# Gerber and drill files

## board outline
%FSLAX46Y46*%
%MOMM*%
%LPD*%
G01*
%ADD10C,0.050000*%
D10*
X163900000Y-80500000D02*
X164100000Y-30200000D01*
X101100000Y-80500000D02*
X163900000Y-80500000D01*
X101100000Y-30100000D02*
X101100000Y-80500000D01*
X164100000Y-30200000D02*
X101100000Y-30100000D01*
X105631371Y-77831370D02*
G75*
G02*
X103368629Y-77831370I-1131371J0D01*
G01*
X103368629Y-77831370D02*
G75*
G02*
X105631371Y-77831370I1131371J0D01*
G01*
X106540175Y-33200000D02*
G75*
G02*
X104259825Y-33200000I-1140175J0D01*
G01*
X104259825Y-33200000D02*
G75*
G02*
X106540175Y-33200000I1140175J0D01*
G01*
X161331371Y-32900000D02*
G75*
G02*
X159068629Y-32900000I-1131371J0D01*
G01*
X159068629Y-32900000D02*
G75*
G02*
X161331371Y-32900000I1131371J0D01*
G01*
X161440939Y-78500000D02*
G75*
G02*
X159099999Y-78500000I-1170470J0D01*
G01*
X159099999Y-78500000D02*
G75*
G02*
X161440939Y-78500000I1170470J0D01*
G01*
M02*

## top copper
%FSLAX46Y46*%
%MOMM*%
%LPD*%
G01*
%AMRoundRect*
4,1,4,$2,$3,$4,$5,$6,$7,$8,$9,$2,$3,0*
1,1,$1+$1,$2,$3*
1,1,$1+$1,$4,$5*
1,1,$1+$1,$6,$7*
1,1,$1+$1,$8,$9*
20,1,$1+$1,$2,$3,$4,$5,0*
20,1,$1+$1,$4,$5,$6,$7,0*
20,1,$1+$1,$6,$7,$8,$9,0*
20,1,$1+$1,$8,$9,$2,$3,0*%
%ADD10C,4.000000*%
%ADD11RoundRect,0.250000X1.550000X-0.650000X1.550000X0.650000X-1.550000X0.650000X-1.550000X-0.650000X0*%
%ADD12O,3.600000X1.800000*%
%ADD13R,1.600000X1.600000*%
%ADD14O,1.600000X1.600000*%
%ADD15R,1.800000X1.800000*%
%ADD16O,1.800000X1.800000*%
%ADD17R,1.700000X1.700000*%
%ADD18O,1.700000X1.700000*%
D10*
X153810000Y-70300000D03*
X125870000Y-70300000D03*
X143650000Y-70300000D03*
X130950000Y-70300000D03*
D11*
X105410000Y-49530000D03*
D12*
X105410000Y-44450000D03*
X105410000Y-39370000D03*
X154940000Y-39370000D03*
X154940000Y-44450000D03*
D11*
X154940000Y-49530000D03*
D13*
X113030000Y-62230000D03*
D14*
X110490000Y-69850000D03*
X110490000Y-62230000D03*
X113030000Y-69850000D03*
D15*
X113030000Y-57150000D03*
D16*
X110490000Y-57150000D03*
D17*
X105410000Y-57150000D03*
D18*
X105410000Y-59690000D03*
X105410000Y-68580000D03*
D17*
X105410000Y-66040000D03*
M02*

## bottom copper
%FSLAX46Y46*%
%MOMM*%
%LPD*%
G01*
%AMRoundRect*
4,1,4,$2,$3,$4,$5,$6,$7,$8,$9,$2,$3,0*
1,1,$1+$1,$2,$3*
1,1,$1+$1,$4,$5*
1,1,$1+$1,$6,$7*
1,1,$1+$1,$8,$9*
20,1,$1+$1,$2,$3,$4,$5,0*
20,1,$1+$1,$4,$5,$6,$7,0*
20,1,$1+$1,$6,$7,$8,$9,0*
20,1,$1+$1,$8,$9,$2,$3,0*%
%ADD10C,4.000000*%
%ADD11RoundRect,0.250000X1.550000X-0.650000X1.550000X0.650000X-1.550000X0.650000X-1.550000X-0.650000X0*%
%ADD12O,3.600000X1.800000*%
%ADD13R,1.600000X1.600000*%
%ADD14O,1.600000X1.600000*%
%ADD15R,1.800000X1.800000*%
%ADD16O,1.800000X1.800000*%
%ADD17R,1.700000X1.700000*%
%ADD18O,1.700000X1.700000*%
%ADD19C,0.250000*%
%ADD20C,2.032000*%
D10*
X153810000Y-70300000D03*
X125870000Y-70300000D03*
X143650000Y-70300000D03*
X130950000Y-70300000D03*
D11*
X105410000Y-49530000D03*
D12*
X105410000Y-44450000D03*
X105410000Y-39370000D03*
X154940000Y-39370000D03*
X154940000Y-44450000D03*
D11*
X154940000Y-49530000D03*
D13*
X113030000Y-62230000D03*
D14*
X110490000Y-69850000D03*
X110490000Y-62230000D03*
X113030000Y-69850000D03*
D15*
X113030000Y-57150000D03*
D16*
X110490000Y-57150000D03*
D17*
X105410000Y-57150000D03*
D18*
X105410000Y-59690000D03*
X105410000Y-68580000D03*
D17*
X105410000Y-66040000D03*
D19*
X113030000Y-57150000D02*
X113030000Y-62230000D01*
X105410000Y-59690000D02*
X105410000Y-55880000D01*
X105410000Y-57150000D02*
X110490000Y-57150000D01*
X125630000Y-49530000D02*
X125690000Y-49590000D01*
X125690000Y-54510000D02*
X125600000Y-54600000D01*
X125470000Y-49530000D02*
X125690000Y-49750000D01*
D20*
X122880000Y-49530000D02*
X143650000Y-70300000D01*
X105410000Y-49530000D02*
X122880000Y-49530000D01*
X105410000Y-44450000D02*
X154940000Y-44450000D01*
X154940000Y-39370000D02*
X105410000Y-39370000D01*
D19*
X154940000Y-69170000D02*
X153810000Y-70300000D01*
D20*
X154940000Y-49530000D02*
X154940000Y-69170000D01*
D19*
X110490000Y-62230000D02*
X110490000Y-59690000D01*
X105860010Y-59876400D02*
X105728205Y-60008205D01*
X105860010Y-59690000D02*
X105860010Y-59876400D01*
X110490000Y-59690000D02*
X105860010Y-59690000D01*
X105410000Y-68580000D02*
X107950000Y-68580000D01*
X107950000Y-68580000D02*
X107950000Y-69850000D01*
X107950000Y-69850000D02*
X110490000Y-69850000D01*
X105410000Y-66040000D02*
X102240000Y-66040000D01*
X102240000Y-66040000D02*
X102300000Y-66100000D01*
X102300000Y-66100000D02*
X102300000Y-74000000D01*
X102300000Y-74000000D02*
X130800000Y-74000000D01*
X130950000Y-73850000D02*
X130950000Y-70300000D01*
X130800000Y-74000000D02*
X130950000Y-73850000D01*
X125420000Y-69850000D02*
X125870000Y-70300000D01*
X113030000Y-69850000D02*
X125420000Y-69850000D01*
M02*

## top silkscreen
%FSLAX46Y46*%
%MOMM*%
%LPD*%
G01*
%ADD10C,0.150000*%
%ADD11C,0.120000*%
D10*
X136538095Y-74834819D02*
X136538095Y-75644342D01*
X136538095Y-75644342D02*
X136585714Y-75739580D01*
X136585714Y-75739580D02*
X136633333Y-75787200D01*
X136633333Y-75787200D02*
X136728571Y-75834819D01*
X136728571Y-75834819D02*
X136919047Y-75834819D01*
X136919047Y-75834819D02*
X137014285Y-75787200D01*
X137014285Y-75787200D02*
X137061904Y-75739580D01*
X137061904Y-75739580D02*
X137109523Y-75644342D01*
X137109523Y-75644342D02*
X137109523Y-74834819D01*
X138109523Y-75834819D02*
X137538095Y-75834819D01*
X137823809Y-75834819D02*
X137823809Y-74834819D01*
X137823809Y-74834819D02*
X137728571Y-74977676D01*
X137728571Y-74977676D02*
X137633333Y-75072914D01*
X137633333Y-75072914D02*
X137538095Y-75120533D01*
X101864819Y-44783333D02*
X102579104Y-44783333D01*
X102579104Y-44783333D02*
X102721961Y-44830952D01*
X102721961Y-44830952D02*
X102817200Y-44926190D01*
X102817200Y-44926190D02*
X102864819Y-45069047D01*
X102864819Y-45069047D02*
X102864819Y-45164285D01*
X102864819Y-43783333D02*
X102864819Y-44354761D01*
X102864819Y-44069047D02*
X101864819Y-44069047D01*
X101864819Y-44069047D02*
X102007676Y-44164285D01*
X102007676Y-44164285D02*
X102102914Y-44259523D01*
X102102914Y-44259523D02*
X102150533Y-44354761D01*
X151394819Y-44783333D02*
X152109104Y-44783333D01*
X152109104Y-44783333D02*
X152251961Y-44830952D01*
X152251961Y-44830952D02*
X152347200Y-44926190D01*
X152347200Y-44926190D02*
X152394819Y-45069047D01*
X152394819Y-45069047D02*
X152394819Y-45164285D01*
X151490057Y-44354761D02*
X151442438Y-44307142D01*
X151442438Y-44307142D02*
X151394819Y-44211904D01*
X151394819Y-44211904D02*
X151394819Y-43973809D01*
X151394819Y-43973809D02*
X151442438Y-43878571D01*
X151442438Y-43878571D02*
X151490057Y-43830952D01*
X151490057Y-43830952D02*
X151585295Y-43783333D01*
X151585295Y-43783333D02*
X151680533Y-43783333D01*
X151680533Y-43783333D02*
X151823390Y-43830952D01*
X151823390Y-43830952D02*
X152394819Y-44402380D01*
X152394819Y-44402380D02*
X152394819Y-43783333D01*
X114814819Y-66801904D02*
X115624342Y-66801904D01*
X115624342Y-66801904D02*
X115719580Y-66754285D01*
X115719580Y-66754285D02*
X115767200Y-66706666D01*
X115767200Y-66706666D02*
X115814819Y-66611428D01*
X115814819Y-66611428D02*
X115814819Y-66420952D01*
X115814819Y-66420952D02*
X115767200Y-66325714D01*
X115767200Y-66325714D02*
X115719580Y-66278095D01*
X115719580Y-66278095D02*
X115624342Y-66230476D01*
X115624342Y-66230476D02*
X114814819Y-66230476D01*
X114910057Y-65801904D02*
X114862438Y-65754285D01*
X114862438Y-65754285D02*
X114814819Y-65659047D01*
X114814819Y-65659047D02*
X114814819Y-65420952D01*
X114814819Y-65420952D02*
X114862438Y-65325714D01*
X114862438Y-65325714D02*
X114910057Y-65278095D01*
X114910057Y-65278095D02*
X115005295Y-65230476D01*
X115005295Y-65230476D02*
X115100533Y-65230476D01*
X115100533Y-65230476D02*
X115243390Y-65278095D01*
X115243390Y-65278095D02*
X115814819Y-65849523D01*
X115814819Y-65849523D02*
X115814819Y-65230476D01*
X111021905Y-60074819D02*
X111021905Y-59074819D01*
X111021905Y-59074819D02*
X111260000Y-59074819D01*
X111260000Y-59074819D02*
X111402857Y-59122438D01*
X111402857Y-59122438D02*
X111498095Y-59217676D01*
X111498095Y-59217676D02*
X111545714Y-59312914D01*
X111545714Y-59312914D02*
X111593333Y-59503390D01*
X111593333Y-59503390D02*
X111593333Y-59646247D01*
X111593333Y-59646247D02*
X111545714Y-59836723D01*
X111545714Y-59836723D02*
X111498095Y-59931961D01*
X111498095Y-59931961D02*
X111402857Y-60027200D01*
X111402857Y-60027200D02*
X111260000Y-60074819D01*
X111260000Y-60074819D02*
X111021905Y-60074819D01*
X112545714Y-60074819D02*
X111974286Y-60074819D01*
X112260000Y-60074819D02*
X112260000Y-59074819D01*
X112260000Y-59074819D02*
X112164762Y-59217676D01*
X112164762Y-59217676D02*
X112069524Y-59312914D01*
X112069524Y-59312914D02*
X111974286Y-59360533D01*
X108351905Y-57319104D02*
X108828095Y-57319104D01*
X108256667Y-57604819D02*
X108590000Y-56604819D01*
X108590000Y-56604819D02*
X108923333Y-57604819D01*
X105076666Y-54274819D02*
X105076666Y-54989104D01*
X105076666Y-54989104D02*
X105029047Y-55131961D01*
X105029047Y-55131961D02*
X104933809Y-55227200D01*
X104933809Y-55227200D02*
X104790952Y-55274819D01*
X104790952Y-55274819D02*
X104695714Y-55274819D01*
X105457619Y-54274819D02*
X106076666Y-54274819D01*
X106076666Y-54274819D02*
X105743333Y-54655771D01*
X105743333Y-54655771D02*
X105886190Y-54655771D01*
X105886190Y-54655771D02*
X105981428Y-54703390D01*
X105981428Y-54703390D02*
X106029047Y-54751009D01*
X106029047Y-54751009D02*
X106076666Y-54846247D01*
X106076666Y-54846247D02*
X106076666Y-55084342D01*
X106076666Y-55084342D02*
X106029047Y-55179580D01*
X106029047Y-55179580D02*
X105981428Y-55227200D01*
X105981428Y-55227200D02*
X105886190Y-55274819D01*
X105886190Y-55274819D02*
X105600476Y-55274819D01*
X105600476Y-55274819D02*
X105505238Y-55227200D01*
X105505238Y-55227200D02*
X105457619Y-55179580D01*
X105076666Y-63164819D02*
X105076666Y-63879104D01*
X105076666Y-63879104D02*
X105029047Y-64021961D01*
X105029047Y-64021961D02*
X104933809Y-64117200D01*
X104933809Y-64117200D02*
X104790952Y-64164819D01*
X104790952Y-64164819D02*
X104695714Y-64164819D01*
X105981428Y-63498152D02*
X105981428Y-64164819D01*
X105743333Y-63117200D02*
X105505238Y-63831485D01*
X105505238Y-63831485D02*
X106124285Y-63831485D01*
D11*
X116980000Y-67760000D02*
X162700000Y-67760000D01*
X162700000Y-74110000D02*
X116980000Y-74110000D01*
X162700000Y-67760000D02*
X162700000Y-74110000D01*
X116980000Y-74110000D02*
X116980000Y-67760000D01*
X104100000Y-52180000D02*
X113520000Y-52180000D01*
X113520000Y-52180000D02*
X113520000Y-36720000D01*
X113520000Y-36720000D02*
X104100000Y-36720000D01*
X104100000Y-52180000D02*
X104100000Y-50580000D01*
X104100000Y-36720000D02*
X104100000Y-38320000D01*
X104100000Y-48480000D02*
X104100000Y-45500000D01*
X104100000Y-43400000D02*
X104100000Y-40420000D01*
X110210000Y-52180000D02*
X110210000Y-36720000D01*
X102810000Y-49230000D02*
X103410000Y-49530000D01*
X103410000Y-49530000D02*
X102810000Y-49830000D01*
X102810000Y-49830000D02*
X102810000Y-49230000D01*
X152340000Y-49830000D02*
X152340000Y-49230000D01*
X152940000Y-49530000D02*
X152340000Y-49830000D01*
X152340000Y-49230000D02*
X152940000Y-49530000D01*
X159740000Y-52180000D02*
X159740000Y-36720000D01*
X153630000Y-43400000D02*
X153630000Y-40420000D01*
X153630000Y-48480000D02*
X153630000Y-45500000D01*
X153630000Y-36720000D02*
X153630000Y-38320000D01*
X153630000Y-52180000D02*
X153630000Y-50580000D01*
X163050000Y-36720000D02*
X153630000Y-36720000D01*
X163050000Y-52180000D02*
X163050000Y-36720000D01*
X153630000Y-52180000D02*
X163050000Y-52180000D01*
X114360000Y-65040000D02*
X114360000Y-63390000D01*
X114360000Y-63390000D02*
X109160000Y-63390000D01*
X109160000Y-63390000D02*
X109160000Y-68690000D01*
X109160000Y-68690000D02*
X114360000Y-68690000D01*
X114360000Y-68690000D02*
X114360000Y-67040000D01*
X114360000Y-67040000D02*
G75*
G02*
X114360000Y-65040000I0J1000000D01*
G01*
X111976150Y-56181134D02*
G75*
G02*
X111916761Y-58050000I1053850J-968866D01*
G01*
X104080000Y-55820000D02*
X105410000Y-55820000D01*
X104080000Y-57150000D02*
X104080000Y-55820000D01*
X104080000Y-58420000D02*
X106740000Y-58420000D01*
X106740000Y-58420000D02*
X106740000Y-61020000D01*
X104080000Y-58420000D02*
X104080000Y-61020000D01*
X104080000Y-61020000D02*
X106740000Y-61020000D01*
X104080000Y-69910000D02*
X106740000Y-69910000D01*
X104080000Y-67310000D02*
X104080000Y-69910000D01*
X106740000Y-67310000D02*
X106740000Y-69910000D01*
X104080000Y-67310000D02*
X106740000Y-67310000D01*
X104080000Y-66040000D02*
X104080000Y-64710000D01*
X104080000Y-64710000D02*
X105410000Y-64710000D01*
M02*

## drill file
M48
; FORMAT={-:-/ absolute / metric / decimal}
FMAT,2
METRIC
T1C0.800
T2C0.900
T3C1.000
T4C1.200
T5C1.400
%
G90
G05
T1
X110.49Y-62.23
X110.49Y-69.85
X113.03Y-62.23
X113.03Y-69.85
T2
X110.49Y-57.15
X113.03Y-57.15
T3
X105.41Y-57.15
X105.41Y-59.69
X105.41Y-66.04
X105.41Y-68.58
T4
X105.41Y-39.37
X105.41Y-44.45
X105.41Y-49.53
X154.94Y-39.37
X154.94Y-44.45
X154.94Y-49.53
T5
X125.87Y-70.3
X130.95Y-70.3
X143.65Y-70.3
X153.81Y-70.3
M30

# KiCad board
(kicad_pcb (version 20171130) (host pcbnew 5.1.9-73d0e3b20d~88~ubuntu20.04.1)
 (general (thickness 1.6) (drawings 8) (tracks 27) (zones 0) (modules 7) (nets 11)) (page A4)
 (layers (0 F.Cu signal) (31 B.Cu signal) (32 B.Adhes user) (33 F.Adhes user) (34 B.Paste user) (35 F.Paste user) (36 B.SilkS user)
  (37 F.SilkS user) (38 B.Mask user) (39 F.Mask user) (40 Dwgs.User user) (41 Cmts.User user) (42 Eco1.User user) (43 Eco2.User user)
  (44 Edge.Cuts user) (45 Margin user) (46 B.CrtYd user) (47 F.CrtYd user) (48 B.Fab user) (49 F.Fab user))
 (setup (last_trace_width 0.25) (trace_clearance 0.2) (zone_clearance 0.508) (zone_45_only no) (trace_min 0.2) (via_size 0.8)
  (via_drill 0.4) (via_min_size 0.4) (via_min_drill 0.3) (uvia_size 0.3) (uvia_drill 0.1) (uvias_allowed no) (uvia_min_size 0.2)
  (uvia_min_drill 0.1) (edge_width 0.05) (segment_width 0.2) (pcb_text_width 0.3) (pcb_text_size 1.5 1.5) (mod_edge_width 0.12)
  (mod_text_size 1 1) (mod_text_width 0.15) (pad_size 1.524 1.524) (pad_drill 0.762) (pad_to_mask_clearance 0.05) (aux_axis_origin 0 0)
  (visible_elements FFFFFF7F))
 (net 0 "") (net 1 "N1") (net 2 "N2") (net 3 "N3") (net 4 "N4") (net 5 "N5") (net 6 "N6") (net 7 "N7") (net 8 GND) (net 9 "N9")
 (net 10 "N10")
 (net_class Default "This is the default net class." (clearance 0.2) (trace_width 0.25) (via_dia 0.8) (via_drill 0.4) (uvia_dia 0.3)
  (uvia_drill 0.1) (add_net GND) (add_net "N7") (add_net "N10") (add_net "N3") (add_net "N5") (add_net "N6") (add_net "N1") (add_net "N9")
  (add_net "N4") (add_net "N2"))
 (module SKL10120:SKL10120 (layer F.Cu) (at 137.3 70.3)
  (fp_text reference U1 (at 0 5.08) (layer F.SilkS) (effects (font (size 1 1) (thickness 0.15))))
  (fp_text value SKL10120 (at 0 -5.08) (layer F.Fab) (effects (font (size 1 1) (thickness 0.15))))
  (fp_line (start -20.32 -2.54) (end 25.4 -2.54) (layer F.SilkS) (width 0.12))
  (fp_line (start 25.4 3.81) (end -20.32 3.81) (layer F.SilkS) (width 0.12))
  (fp_line (start 25.4 -2.54) (end 25.4 3.81) (layer F.SilkS) (width 0.12))
  (fp_line (start -20.32 3.81) (end -20.32 -2.54) (layer F.SilkS) (width 0.12))
  (pad 1 thru_hole circle (at 16.51 0) (size 4 4) (drill 1.4) (layers *.Cu *.Mask) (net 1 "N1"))
  (pad 4 thru_hole circle (at -11.43 0) (size 4 4) (drill 1.4) (layers *.Cu *.Mask) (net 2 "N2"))
  (pad 2 thru_hole circle (at 6.35 0) (size 4 4) (drill 1.4) (layers *.Cu *.Mask) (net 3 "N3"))
  (pad 3 thru_hole circle (at -6.35 0) (size 4 4) (drill 1.4) (layers *.Cu *.Mask) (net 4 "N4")))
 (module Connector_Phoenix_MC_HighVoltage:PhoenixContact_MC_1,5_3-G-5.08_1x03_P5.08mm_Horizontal (layer F.Cu) (at 105.41 49.53 90)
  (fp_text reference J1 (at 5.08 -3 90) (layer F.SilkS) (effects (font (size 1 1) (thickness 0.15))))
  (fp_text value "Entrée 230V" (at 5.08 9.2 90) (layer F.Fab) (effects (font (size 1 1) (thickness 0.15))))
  (fp_line (start -2.65 -1.31) (end -2.65 8.11) (layer F.SilkS) (width 0.12))
  (fp_line (start -2.65 8.11) (end 12.81 8.11) (layer F.SilkS) (width 0.12))
  (fp_line (start 12.81 8.11) (end 12.81 -1.31) (layer F.SilkS) (width 0.12))
  (fp_line (start -2.65 -1.31) (end -1.05 -1.31) (layer F.SilkS) (width 0.12))
  (fp_line (start 12.81 -1.31) (end 11.21 -1.31) (layer F.SilkS) (width 0.12))
  (fp_line (start 1.05 -1.31) (end 4.03 -1.31) (layer F.SilkS) (width 0.12))
  (fp_line (start 6.13 -1.31) (end 9.11 -1.31) (layer F.SilkS) (width 0.12))
  (fp_line (start -2.65 4.8) (end 12.81 4.8) (layer F.SilkS) (width 0.12))
  (fp_line (start 0.3 -2.6) (end 0 -2) (layer F.SilkS) (width 0.12))
  (fp_line (start 0 -2) (end -0.3 -2.6) (layer F.SilkS) (width 0.12))
  (fp_line (start -0.3 -2.6) (end 0.3 -2.6) (layer F.SilkS) (width 0.12))
  (pad 1 thru_hole roundrect (at 0 0 90) (size 1.8 3.6) (drill 1.2) (layers *.Cu *.Mask) (roundrect_rratio 0.138889) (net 3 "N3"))
  (pad 2 thru_hole oval (at 5.08 0 90) (size 1.8 3.6) (drill 1.2) (layers *.Cu *.Mask) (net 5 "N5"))
  (pad 3 thru_hole oval (at 10.16 0 90) (size 1.8 3.6) (drill 1.2) (layers *.Cu *.Mask) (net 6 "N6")))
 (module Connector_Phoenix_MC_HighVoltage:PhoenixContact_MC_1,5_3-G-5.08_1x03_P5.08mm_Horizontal (layer F.Cu) (at 154.94 49.53 90)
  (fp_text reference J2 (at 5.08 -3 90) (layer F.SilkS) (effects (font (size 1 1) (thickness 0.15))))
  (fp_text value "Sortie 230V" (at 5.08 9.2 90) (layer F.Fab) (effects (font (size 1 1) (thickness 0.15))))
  (fp_line (start -0.3 -2.6) (end 0.3 -2.6) (layer F.SilkS) (width 0.12))
  (fp_line (start 0 -2) (end -0.3 -2.6) (layer F.SilkS) (width 0.12))
  (fp_line (start 0.3 -2.6) (end 0 -2) (layer F.SilkS) (width 0.12))
  (fp_line (start -2.65 4.8) (end 12.81 4.8) (layer F.SilkS) (width 0.12))
  (fp_line (start 6.13 -1.31) (end 9.11 -1.31) (layer F.SilkS) (width 0.12))
  (fp_line (start 1.05 -1.31) (end 4.03 -1.31) (layer F.SilkS) (width 0.12))
  (fp_line (start 12.81 -1.31) (end 11.21 -1.31) (layer F.SilkS) (width 0.12))
  (fp_line (start -2.65 -1.31) (end -1.05 -1.31) (layer F.SilkS) (width 0.12))
  (fp_line (start 12.81 8.11) (end 12.81 -1.31) (layer F.SilkS) (width 0.12))
  (fp_line (start -2.65 8.11) (end 12.81 8.11) (layer F.SilkS) (width 0.12))
  (fp_line (start -2.65 -1.31) (end -2.65 8.11) (layer F.SilkS) (width 0.12))
  (pad 3 thru_hole oval (at 10.16 0 90) (size 1.8 3.6) (drill 1.2) (layers *.Cu *.Mask) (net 6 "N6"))
  (pad 2 thru_hole oval (at 5.08 0 90) (size 1.8 3.6) (drill 1.2) (layers *.Cu *.Mask) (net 5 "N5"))
  (pad 1 thru_hole roundrect (at 0 0 90) (size 1.8 3.6) (drill 1.2) (layers *.Cu *.Mask) (roundrect_rratio 0.138889) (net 1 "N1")))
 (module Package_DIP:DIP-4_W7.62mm (layer F.Cu) (at 113.03 62.23 270)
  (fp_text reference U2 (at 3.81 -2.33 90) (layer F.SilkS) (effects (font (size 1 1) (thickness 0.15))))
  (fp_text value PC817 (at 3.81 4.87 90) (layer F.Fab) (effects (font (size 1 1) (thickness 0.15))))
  (fp_line (start 2.81 -1.33) (end 1.16 -1.33) (layer F.SilkS) (width 0.12))
  (fp_line (start 1.16 -1.33) (end 1.16 3.87) (layer F.SilkS) (width 0.12))
  (fp_line (start 1.16 3.87) (end 6.46 3.87) (layer F.SilkS) (width 0.12))
  (fp_line (start 6.46 3.87) (end 6.46 -1.33) (layer F.SilkS) (width 0.12))
  (fp_line (start 6.46 -1.33) (end 4.81 -1.33) (layer F.SilkS) (width 0.12))
  (fp_arc (start 3.81 -1.33) (end 2.81 -1.33) (angle -180) (layer F.SilkS) (width 0.12))
  (pad 1 thru_hole rect (at 0 0 270) (size 1.6 1.6) (drill 0.8) (layers *.Cu *.Mask) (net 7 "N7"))
  (pad 3 thru_hole oval (at 7.62 2.54 270) (size 1.6 1.6) (drill 0.8) (layers *.Cu *.Mask) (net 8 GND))
  (pad 2 thru_hole oval (at 0 2.54 270) (size 1.6 1.6) (drill 0.8) (layers *.Cu *.Mask) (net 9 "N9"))
  (pad 4 thru_hole oval (at 7.62 0 270) (size 1.6 1.6) (drill 0.8) (layers *.Cu *.Mask) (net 2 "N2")))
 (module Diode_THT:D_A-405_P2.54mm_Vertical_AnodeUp (layer F.Cu) (at 113.03 57.15 180)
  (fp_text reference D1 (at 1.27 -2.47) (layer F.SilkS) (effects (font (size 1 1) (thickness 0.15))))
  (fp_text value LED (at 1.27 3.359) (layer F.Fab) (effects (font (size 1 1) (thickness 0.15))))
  (fp_arc (start 0 0) (end 1.113239 -0.9) (angle -278.451986) (layer F.SilkS) (width 0.12))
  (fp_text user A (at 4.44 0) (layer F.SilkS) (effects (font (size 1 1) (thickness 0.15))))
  (pad 1 thru_hole rect (at 0 0 180) (size 1.8 1.8) (drill 0.9) (layers *.Cu *.Mask) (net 7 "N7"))
  (pad 2 thru_hole oval (at 2.54 0 180) (size 1.8 1.8) (drill 0.9) (layers *.Cu *.Mask) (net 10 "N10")))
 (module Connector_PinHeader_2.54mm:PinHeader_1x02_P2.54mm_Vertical (layer F.Cu) (at 105.41 57.15)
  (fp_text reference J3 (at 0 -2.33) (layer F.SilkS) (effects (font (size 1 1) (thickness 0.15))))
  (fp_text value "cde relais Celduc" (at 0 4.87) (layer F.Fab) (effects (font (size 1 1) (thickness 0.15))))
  (fp_line (start -1.33 -1.33) (end 0 -1.33) (layer F.SilkS) (width 0.12))
  (fp_line (start -1.33 0) (end -1.33 -1.33) (layer F.SilkS) (width 0.12))
  (fp_line (start -1.33 1.27) (end 1.33 1.27) (layer F.SilkS) (width 0.12))
  (fp_line (start 1.33 1.27) (end 1.33 3.87) (layer F.SilkS) (width 0.12))
  (fp_line (start -1.33 1.27) (end -1.33 3.87) (layer F.SilkS) (width 0.12))
  (fp_line (start -1.33 3.87) (end 1.33 3.87) (layer F.SilkS) (width 0.12))
  (pad 1 thru_hole rect (at 0 0) (size 1.7 1.7) (drill 1) (layers *.Cu *.Mask) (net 10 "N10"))
  (pad 2 thru_hole oval (at 0 2.54) (size 1.7 1.7) (drill 1) (layers *.Cu *.Mask) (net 9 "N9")))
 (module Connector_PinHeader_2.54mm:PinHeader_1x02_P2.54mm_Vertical (layer F.Cu) (at 105.41 66.04)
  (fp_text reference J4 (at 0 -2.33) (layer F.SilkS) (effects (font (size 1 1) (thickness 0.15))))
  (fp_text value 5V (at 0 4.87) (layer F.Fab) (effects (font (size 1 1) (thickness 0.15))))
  (fp_line (start -1.33 3.87) (end 1.33 3.87) (layer F.SilkS) (width 0.12))
  (fp_line (start -1.33 1.27) (end -1.33 3.87) (layer F.SilkS) (width 0.12))
  (fp_line (start 1.33 1.27) (end 1.33 3.87) (layer F.SilkS) (width 0.12))
  (fp_line (start -1.33 1.27) (end 1.33 1.27) (layer F.SilkS) (width 0.12))
  (fp_line (start -1.33 0) (end -1.33 -1.33) (layer F.SilkS) (width 0.12))
  (fp_line (start -1.33 -1.33) (end 0 -1.33) (layer F.SilkS) (width 0.12))
  (pad 2 thru_hole oval (at 0 2.54) (size 1.7 1.7) (drill 1) (layers *.Cu *.Mask) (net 8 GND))
  (pad 1 thru_hole rect (at 0 0) (size 1.7 1.7) (drill 1) (layers *.Cu *.Mask) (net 4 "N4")))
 (gr_line (start 163.9 80.5) (end 164.1 30.2) (layer Edge.Cuts) (width 0.05))
 (gr_line (start 101.1 80.5) (end 163.9 80.5) (layer Edge.Cuts) (width 0.05))
 (gr_line (start 101.1 30.1) (end 101.1 80.5) (layer Edge.Cuts) (width 0.05))
 (gr_line (start 164.1 30.2) (end 101.1 30.1) (layer Edge.Cuts) (width 0.05))
 (gr_circle (center 104.5 77.83137) (end 105.3 77.03137) (layer Edge.Cuts) (width 0.05))
 (gr_circle (center 105.4 33.2) (end 106.3 33.9) (layer Edge.Cuts) (width 0.05))
 (gr_circle (center 160.2 32.9) (end 159.4 33.7) (layer Edge.Cuts) (width 0.05))
 (gr_circle (center 160.270469 78.5) (end 159.170469 78.9) (layer Edge.Cuts) (width 0.05))
 (segment (start 113.03 57.15) (end 113.03 62.23) (width 0.25) (layer B.Cu) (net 7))
 (segment (start 105.41 59.69) (end 105.41 55.88) (width 0.25) (layer B.Cu) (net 10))
 (segment (start 105.41 57.15) (end 110.49 57.15) (width 0.25) (layer B.Cu) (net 10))
 (segment (start 125.63 49.53) (end 125.69 49.59) (width 0.25) (layer B.Cu) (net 3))
 (segment (start 125.69 54.51) (end 125.6 54.6) (width 0.25) (layer B.Cu) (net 3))
 (segment (start 125.47 49.53) (end 125.69 49.75) (width 0.25) (layer B.Cu) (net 3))
 (segment (start 122.88 49.53) (end 143.65 70.3) (width 2.032) (layer B.Cu) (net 3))
 (segment (start 105.41 49.53) (end 122.88 49.53) (width 2.032) (layer B.Cu) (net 3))
 (segment (start 105.41 44.45) (end 154.94 44.45) (width 2.032) (layer B.Cu) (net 5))
 (segment (start 154.94 39.37) (end 105.41 39.37) (width 2.032) (layer B.Cu) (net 6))
 (segment (start 154.94 69.17) (end 153.81 70.3) (width 0.25) (layer B.Cu) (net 1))
 (segment (start 154.94 49.53) (end 154.94 69.17) (width 2.032) (layer B.Cu) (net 1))
 (segment (start 110.49 62.23) (end 110.49 59.69) (width 0.25) (layer B.Cu) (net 9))
 (segment (start 105.86001 59.8764) (end 105.728205 60.008205) (width 0.25) (layer B.Cu) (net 9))
 (segment (start 105.86001 59.69) (end 105.86001 59.8764) (width 0.25) (layer B.Cu) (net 9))
 (segment (start 110.49 59.69) (end 105.86001 59.69) (width 0.25) (layer B.Cu) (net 9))
 (segment (start 105.41 68.58) (end 107.95 68.58) (width 0.25) (layer B.Cu) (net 8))
 (segment (start 107.95 68.58) (end 107.95 69.85) (width 0.25) (layer B.Cu) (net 8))
 (segment (start 107.95 69.85) (end 110.49 69.85) (width 0.25) (layer B.Cu) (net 8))
 (segment (start 105.41 66.04) (end 102.24 66.04) (width 0.25) (layer B.Cu) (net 4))
 (segment (start 102.24 66.04) (end 102.3 66.1) (width 0.25) (layer B.Cu) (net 4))
 (segment (start 102.3 66.1) (end 102.3 74) (width 0.25) (layer B.Cu) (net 4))
 (segment (start 102.3 74) (end 130.8 74) (width 0.25) (layer B.Cu) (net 4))
 (segment (start 130.95 73.85) (end 130.95 70.3) (width 0.25) (layer B.Cu) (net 4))
 (segment (start 130.8 74) (end 130.95 73.85) (width 0.25) (layer B.Cu) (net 4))
 (segment (start 125.42 69.85) (end 125.87 70.3) (width 0.25) (layer B.Cu) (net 2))
 (segment (start 113.03 69.85) (end 125.42 69.85) (width 0.25) (layer B.Cu) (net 2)))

